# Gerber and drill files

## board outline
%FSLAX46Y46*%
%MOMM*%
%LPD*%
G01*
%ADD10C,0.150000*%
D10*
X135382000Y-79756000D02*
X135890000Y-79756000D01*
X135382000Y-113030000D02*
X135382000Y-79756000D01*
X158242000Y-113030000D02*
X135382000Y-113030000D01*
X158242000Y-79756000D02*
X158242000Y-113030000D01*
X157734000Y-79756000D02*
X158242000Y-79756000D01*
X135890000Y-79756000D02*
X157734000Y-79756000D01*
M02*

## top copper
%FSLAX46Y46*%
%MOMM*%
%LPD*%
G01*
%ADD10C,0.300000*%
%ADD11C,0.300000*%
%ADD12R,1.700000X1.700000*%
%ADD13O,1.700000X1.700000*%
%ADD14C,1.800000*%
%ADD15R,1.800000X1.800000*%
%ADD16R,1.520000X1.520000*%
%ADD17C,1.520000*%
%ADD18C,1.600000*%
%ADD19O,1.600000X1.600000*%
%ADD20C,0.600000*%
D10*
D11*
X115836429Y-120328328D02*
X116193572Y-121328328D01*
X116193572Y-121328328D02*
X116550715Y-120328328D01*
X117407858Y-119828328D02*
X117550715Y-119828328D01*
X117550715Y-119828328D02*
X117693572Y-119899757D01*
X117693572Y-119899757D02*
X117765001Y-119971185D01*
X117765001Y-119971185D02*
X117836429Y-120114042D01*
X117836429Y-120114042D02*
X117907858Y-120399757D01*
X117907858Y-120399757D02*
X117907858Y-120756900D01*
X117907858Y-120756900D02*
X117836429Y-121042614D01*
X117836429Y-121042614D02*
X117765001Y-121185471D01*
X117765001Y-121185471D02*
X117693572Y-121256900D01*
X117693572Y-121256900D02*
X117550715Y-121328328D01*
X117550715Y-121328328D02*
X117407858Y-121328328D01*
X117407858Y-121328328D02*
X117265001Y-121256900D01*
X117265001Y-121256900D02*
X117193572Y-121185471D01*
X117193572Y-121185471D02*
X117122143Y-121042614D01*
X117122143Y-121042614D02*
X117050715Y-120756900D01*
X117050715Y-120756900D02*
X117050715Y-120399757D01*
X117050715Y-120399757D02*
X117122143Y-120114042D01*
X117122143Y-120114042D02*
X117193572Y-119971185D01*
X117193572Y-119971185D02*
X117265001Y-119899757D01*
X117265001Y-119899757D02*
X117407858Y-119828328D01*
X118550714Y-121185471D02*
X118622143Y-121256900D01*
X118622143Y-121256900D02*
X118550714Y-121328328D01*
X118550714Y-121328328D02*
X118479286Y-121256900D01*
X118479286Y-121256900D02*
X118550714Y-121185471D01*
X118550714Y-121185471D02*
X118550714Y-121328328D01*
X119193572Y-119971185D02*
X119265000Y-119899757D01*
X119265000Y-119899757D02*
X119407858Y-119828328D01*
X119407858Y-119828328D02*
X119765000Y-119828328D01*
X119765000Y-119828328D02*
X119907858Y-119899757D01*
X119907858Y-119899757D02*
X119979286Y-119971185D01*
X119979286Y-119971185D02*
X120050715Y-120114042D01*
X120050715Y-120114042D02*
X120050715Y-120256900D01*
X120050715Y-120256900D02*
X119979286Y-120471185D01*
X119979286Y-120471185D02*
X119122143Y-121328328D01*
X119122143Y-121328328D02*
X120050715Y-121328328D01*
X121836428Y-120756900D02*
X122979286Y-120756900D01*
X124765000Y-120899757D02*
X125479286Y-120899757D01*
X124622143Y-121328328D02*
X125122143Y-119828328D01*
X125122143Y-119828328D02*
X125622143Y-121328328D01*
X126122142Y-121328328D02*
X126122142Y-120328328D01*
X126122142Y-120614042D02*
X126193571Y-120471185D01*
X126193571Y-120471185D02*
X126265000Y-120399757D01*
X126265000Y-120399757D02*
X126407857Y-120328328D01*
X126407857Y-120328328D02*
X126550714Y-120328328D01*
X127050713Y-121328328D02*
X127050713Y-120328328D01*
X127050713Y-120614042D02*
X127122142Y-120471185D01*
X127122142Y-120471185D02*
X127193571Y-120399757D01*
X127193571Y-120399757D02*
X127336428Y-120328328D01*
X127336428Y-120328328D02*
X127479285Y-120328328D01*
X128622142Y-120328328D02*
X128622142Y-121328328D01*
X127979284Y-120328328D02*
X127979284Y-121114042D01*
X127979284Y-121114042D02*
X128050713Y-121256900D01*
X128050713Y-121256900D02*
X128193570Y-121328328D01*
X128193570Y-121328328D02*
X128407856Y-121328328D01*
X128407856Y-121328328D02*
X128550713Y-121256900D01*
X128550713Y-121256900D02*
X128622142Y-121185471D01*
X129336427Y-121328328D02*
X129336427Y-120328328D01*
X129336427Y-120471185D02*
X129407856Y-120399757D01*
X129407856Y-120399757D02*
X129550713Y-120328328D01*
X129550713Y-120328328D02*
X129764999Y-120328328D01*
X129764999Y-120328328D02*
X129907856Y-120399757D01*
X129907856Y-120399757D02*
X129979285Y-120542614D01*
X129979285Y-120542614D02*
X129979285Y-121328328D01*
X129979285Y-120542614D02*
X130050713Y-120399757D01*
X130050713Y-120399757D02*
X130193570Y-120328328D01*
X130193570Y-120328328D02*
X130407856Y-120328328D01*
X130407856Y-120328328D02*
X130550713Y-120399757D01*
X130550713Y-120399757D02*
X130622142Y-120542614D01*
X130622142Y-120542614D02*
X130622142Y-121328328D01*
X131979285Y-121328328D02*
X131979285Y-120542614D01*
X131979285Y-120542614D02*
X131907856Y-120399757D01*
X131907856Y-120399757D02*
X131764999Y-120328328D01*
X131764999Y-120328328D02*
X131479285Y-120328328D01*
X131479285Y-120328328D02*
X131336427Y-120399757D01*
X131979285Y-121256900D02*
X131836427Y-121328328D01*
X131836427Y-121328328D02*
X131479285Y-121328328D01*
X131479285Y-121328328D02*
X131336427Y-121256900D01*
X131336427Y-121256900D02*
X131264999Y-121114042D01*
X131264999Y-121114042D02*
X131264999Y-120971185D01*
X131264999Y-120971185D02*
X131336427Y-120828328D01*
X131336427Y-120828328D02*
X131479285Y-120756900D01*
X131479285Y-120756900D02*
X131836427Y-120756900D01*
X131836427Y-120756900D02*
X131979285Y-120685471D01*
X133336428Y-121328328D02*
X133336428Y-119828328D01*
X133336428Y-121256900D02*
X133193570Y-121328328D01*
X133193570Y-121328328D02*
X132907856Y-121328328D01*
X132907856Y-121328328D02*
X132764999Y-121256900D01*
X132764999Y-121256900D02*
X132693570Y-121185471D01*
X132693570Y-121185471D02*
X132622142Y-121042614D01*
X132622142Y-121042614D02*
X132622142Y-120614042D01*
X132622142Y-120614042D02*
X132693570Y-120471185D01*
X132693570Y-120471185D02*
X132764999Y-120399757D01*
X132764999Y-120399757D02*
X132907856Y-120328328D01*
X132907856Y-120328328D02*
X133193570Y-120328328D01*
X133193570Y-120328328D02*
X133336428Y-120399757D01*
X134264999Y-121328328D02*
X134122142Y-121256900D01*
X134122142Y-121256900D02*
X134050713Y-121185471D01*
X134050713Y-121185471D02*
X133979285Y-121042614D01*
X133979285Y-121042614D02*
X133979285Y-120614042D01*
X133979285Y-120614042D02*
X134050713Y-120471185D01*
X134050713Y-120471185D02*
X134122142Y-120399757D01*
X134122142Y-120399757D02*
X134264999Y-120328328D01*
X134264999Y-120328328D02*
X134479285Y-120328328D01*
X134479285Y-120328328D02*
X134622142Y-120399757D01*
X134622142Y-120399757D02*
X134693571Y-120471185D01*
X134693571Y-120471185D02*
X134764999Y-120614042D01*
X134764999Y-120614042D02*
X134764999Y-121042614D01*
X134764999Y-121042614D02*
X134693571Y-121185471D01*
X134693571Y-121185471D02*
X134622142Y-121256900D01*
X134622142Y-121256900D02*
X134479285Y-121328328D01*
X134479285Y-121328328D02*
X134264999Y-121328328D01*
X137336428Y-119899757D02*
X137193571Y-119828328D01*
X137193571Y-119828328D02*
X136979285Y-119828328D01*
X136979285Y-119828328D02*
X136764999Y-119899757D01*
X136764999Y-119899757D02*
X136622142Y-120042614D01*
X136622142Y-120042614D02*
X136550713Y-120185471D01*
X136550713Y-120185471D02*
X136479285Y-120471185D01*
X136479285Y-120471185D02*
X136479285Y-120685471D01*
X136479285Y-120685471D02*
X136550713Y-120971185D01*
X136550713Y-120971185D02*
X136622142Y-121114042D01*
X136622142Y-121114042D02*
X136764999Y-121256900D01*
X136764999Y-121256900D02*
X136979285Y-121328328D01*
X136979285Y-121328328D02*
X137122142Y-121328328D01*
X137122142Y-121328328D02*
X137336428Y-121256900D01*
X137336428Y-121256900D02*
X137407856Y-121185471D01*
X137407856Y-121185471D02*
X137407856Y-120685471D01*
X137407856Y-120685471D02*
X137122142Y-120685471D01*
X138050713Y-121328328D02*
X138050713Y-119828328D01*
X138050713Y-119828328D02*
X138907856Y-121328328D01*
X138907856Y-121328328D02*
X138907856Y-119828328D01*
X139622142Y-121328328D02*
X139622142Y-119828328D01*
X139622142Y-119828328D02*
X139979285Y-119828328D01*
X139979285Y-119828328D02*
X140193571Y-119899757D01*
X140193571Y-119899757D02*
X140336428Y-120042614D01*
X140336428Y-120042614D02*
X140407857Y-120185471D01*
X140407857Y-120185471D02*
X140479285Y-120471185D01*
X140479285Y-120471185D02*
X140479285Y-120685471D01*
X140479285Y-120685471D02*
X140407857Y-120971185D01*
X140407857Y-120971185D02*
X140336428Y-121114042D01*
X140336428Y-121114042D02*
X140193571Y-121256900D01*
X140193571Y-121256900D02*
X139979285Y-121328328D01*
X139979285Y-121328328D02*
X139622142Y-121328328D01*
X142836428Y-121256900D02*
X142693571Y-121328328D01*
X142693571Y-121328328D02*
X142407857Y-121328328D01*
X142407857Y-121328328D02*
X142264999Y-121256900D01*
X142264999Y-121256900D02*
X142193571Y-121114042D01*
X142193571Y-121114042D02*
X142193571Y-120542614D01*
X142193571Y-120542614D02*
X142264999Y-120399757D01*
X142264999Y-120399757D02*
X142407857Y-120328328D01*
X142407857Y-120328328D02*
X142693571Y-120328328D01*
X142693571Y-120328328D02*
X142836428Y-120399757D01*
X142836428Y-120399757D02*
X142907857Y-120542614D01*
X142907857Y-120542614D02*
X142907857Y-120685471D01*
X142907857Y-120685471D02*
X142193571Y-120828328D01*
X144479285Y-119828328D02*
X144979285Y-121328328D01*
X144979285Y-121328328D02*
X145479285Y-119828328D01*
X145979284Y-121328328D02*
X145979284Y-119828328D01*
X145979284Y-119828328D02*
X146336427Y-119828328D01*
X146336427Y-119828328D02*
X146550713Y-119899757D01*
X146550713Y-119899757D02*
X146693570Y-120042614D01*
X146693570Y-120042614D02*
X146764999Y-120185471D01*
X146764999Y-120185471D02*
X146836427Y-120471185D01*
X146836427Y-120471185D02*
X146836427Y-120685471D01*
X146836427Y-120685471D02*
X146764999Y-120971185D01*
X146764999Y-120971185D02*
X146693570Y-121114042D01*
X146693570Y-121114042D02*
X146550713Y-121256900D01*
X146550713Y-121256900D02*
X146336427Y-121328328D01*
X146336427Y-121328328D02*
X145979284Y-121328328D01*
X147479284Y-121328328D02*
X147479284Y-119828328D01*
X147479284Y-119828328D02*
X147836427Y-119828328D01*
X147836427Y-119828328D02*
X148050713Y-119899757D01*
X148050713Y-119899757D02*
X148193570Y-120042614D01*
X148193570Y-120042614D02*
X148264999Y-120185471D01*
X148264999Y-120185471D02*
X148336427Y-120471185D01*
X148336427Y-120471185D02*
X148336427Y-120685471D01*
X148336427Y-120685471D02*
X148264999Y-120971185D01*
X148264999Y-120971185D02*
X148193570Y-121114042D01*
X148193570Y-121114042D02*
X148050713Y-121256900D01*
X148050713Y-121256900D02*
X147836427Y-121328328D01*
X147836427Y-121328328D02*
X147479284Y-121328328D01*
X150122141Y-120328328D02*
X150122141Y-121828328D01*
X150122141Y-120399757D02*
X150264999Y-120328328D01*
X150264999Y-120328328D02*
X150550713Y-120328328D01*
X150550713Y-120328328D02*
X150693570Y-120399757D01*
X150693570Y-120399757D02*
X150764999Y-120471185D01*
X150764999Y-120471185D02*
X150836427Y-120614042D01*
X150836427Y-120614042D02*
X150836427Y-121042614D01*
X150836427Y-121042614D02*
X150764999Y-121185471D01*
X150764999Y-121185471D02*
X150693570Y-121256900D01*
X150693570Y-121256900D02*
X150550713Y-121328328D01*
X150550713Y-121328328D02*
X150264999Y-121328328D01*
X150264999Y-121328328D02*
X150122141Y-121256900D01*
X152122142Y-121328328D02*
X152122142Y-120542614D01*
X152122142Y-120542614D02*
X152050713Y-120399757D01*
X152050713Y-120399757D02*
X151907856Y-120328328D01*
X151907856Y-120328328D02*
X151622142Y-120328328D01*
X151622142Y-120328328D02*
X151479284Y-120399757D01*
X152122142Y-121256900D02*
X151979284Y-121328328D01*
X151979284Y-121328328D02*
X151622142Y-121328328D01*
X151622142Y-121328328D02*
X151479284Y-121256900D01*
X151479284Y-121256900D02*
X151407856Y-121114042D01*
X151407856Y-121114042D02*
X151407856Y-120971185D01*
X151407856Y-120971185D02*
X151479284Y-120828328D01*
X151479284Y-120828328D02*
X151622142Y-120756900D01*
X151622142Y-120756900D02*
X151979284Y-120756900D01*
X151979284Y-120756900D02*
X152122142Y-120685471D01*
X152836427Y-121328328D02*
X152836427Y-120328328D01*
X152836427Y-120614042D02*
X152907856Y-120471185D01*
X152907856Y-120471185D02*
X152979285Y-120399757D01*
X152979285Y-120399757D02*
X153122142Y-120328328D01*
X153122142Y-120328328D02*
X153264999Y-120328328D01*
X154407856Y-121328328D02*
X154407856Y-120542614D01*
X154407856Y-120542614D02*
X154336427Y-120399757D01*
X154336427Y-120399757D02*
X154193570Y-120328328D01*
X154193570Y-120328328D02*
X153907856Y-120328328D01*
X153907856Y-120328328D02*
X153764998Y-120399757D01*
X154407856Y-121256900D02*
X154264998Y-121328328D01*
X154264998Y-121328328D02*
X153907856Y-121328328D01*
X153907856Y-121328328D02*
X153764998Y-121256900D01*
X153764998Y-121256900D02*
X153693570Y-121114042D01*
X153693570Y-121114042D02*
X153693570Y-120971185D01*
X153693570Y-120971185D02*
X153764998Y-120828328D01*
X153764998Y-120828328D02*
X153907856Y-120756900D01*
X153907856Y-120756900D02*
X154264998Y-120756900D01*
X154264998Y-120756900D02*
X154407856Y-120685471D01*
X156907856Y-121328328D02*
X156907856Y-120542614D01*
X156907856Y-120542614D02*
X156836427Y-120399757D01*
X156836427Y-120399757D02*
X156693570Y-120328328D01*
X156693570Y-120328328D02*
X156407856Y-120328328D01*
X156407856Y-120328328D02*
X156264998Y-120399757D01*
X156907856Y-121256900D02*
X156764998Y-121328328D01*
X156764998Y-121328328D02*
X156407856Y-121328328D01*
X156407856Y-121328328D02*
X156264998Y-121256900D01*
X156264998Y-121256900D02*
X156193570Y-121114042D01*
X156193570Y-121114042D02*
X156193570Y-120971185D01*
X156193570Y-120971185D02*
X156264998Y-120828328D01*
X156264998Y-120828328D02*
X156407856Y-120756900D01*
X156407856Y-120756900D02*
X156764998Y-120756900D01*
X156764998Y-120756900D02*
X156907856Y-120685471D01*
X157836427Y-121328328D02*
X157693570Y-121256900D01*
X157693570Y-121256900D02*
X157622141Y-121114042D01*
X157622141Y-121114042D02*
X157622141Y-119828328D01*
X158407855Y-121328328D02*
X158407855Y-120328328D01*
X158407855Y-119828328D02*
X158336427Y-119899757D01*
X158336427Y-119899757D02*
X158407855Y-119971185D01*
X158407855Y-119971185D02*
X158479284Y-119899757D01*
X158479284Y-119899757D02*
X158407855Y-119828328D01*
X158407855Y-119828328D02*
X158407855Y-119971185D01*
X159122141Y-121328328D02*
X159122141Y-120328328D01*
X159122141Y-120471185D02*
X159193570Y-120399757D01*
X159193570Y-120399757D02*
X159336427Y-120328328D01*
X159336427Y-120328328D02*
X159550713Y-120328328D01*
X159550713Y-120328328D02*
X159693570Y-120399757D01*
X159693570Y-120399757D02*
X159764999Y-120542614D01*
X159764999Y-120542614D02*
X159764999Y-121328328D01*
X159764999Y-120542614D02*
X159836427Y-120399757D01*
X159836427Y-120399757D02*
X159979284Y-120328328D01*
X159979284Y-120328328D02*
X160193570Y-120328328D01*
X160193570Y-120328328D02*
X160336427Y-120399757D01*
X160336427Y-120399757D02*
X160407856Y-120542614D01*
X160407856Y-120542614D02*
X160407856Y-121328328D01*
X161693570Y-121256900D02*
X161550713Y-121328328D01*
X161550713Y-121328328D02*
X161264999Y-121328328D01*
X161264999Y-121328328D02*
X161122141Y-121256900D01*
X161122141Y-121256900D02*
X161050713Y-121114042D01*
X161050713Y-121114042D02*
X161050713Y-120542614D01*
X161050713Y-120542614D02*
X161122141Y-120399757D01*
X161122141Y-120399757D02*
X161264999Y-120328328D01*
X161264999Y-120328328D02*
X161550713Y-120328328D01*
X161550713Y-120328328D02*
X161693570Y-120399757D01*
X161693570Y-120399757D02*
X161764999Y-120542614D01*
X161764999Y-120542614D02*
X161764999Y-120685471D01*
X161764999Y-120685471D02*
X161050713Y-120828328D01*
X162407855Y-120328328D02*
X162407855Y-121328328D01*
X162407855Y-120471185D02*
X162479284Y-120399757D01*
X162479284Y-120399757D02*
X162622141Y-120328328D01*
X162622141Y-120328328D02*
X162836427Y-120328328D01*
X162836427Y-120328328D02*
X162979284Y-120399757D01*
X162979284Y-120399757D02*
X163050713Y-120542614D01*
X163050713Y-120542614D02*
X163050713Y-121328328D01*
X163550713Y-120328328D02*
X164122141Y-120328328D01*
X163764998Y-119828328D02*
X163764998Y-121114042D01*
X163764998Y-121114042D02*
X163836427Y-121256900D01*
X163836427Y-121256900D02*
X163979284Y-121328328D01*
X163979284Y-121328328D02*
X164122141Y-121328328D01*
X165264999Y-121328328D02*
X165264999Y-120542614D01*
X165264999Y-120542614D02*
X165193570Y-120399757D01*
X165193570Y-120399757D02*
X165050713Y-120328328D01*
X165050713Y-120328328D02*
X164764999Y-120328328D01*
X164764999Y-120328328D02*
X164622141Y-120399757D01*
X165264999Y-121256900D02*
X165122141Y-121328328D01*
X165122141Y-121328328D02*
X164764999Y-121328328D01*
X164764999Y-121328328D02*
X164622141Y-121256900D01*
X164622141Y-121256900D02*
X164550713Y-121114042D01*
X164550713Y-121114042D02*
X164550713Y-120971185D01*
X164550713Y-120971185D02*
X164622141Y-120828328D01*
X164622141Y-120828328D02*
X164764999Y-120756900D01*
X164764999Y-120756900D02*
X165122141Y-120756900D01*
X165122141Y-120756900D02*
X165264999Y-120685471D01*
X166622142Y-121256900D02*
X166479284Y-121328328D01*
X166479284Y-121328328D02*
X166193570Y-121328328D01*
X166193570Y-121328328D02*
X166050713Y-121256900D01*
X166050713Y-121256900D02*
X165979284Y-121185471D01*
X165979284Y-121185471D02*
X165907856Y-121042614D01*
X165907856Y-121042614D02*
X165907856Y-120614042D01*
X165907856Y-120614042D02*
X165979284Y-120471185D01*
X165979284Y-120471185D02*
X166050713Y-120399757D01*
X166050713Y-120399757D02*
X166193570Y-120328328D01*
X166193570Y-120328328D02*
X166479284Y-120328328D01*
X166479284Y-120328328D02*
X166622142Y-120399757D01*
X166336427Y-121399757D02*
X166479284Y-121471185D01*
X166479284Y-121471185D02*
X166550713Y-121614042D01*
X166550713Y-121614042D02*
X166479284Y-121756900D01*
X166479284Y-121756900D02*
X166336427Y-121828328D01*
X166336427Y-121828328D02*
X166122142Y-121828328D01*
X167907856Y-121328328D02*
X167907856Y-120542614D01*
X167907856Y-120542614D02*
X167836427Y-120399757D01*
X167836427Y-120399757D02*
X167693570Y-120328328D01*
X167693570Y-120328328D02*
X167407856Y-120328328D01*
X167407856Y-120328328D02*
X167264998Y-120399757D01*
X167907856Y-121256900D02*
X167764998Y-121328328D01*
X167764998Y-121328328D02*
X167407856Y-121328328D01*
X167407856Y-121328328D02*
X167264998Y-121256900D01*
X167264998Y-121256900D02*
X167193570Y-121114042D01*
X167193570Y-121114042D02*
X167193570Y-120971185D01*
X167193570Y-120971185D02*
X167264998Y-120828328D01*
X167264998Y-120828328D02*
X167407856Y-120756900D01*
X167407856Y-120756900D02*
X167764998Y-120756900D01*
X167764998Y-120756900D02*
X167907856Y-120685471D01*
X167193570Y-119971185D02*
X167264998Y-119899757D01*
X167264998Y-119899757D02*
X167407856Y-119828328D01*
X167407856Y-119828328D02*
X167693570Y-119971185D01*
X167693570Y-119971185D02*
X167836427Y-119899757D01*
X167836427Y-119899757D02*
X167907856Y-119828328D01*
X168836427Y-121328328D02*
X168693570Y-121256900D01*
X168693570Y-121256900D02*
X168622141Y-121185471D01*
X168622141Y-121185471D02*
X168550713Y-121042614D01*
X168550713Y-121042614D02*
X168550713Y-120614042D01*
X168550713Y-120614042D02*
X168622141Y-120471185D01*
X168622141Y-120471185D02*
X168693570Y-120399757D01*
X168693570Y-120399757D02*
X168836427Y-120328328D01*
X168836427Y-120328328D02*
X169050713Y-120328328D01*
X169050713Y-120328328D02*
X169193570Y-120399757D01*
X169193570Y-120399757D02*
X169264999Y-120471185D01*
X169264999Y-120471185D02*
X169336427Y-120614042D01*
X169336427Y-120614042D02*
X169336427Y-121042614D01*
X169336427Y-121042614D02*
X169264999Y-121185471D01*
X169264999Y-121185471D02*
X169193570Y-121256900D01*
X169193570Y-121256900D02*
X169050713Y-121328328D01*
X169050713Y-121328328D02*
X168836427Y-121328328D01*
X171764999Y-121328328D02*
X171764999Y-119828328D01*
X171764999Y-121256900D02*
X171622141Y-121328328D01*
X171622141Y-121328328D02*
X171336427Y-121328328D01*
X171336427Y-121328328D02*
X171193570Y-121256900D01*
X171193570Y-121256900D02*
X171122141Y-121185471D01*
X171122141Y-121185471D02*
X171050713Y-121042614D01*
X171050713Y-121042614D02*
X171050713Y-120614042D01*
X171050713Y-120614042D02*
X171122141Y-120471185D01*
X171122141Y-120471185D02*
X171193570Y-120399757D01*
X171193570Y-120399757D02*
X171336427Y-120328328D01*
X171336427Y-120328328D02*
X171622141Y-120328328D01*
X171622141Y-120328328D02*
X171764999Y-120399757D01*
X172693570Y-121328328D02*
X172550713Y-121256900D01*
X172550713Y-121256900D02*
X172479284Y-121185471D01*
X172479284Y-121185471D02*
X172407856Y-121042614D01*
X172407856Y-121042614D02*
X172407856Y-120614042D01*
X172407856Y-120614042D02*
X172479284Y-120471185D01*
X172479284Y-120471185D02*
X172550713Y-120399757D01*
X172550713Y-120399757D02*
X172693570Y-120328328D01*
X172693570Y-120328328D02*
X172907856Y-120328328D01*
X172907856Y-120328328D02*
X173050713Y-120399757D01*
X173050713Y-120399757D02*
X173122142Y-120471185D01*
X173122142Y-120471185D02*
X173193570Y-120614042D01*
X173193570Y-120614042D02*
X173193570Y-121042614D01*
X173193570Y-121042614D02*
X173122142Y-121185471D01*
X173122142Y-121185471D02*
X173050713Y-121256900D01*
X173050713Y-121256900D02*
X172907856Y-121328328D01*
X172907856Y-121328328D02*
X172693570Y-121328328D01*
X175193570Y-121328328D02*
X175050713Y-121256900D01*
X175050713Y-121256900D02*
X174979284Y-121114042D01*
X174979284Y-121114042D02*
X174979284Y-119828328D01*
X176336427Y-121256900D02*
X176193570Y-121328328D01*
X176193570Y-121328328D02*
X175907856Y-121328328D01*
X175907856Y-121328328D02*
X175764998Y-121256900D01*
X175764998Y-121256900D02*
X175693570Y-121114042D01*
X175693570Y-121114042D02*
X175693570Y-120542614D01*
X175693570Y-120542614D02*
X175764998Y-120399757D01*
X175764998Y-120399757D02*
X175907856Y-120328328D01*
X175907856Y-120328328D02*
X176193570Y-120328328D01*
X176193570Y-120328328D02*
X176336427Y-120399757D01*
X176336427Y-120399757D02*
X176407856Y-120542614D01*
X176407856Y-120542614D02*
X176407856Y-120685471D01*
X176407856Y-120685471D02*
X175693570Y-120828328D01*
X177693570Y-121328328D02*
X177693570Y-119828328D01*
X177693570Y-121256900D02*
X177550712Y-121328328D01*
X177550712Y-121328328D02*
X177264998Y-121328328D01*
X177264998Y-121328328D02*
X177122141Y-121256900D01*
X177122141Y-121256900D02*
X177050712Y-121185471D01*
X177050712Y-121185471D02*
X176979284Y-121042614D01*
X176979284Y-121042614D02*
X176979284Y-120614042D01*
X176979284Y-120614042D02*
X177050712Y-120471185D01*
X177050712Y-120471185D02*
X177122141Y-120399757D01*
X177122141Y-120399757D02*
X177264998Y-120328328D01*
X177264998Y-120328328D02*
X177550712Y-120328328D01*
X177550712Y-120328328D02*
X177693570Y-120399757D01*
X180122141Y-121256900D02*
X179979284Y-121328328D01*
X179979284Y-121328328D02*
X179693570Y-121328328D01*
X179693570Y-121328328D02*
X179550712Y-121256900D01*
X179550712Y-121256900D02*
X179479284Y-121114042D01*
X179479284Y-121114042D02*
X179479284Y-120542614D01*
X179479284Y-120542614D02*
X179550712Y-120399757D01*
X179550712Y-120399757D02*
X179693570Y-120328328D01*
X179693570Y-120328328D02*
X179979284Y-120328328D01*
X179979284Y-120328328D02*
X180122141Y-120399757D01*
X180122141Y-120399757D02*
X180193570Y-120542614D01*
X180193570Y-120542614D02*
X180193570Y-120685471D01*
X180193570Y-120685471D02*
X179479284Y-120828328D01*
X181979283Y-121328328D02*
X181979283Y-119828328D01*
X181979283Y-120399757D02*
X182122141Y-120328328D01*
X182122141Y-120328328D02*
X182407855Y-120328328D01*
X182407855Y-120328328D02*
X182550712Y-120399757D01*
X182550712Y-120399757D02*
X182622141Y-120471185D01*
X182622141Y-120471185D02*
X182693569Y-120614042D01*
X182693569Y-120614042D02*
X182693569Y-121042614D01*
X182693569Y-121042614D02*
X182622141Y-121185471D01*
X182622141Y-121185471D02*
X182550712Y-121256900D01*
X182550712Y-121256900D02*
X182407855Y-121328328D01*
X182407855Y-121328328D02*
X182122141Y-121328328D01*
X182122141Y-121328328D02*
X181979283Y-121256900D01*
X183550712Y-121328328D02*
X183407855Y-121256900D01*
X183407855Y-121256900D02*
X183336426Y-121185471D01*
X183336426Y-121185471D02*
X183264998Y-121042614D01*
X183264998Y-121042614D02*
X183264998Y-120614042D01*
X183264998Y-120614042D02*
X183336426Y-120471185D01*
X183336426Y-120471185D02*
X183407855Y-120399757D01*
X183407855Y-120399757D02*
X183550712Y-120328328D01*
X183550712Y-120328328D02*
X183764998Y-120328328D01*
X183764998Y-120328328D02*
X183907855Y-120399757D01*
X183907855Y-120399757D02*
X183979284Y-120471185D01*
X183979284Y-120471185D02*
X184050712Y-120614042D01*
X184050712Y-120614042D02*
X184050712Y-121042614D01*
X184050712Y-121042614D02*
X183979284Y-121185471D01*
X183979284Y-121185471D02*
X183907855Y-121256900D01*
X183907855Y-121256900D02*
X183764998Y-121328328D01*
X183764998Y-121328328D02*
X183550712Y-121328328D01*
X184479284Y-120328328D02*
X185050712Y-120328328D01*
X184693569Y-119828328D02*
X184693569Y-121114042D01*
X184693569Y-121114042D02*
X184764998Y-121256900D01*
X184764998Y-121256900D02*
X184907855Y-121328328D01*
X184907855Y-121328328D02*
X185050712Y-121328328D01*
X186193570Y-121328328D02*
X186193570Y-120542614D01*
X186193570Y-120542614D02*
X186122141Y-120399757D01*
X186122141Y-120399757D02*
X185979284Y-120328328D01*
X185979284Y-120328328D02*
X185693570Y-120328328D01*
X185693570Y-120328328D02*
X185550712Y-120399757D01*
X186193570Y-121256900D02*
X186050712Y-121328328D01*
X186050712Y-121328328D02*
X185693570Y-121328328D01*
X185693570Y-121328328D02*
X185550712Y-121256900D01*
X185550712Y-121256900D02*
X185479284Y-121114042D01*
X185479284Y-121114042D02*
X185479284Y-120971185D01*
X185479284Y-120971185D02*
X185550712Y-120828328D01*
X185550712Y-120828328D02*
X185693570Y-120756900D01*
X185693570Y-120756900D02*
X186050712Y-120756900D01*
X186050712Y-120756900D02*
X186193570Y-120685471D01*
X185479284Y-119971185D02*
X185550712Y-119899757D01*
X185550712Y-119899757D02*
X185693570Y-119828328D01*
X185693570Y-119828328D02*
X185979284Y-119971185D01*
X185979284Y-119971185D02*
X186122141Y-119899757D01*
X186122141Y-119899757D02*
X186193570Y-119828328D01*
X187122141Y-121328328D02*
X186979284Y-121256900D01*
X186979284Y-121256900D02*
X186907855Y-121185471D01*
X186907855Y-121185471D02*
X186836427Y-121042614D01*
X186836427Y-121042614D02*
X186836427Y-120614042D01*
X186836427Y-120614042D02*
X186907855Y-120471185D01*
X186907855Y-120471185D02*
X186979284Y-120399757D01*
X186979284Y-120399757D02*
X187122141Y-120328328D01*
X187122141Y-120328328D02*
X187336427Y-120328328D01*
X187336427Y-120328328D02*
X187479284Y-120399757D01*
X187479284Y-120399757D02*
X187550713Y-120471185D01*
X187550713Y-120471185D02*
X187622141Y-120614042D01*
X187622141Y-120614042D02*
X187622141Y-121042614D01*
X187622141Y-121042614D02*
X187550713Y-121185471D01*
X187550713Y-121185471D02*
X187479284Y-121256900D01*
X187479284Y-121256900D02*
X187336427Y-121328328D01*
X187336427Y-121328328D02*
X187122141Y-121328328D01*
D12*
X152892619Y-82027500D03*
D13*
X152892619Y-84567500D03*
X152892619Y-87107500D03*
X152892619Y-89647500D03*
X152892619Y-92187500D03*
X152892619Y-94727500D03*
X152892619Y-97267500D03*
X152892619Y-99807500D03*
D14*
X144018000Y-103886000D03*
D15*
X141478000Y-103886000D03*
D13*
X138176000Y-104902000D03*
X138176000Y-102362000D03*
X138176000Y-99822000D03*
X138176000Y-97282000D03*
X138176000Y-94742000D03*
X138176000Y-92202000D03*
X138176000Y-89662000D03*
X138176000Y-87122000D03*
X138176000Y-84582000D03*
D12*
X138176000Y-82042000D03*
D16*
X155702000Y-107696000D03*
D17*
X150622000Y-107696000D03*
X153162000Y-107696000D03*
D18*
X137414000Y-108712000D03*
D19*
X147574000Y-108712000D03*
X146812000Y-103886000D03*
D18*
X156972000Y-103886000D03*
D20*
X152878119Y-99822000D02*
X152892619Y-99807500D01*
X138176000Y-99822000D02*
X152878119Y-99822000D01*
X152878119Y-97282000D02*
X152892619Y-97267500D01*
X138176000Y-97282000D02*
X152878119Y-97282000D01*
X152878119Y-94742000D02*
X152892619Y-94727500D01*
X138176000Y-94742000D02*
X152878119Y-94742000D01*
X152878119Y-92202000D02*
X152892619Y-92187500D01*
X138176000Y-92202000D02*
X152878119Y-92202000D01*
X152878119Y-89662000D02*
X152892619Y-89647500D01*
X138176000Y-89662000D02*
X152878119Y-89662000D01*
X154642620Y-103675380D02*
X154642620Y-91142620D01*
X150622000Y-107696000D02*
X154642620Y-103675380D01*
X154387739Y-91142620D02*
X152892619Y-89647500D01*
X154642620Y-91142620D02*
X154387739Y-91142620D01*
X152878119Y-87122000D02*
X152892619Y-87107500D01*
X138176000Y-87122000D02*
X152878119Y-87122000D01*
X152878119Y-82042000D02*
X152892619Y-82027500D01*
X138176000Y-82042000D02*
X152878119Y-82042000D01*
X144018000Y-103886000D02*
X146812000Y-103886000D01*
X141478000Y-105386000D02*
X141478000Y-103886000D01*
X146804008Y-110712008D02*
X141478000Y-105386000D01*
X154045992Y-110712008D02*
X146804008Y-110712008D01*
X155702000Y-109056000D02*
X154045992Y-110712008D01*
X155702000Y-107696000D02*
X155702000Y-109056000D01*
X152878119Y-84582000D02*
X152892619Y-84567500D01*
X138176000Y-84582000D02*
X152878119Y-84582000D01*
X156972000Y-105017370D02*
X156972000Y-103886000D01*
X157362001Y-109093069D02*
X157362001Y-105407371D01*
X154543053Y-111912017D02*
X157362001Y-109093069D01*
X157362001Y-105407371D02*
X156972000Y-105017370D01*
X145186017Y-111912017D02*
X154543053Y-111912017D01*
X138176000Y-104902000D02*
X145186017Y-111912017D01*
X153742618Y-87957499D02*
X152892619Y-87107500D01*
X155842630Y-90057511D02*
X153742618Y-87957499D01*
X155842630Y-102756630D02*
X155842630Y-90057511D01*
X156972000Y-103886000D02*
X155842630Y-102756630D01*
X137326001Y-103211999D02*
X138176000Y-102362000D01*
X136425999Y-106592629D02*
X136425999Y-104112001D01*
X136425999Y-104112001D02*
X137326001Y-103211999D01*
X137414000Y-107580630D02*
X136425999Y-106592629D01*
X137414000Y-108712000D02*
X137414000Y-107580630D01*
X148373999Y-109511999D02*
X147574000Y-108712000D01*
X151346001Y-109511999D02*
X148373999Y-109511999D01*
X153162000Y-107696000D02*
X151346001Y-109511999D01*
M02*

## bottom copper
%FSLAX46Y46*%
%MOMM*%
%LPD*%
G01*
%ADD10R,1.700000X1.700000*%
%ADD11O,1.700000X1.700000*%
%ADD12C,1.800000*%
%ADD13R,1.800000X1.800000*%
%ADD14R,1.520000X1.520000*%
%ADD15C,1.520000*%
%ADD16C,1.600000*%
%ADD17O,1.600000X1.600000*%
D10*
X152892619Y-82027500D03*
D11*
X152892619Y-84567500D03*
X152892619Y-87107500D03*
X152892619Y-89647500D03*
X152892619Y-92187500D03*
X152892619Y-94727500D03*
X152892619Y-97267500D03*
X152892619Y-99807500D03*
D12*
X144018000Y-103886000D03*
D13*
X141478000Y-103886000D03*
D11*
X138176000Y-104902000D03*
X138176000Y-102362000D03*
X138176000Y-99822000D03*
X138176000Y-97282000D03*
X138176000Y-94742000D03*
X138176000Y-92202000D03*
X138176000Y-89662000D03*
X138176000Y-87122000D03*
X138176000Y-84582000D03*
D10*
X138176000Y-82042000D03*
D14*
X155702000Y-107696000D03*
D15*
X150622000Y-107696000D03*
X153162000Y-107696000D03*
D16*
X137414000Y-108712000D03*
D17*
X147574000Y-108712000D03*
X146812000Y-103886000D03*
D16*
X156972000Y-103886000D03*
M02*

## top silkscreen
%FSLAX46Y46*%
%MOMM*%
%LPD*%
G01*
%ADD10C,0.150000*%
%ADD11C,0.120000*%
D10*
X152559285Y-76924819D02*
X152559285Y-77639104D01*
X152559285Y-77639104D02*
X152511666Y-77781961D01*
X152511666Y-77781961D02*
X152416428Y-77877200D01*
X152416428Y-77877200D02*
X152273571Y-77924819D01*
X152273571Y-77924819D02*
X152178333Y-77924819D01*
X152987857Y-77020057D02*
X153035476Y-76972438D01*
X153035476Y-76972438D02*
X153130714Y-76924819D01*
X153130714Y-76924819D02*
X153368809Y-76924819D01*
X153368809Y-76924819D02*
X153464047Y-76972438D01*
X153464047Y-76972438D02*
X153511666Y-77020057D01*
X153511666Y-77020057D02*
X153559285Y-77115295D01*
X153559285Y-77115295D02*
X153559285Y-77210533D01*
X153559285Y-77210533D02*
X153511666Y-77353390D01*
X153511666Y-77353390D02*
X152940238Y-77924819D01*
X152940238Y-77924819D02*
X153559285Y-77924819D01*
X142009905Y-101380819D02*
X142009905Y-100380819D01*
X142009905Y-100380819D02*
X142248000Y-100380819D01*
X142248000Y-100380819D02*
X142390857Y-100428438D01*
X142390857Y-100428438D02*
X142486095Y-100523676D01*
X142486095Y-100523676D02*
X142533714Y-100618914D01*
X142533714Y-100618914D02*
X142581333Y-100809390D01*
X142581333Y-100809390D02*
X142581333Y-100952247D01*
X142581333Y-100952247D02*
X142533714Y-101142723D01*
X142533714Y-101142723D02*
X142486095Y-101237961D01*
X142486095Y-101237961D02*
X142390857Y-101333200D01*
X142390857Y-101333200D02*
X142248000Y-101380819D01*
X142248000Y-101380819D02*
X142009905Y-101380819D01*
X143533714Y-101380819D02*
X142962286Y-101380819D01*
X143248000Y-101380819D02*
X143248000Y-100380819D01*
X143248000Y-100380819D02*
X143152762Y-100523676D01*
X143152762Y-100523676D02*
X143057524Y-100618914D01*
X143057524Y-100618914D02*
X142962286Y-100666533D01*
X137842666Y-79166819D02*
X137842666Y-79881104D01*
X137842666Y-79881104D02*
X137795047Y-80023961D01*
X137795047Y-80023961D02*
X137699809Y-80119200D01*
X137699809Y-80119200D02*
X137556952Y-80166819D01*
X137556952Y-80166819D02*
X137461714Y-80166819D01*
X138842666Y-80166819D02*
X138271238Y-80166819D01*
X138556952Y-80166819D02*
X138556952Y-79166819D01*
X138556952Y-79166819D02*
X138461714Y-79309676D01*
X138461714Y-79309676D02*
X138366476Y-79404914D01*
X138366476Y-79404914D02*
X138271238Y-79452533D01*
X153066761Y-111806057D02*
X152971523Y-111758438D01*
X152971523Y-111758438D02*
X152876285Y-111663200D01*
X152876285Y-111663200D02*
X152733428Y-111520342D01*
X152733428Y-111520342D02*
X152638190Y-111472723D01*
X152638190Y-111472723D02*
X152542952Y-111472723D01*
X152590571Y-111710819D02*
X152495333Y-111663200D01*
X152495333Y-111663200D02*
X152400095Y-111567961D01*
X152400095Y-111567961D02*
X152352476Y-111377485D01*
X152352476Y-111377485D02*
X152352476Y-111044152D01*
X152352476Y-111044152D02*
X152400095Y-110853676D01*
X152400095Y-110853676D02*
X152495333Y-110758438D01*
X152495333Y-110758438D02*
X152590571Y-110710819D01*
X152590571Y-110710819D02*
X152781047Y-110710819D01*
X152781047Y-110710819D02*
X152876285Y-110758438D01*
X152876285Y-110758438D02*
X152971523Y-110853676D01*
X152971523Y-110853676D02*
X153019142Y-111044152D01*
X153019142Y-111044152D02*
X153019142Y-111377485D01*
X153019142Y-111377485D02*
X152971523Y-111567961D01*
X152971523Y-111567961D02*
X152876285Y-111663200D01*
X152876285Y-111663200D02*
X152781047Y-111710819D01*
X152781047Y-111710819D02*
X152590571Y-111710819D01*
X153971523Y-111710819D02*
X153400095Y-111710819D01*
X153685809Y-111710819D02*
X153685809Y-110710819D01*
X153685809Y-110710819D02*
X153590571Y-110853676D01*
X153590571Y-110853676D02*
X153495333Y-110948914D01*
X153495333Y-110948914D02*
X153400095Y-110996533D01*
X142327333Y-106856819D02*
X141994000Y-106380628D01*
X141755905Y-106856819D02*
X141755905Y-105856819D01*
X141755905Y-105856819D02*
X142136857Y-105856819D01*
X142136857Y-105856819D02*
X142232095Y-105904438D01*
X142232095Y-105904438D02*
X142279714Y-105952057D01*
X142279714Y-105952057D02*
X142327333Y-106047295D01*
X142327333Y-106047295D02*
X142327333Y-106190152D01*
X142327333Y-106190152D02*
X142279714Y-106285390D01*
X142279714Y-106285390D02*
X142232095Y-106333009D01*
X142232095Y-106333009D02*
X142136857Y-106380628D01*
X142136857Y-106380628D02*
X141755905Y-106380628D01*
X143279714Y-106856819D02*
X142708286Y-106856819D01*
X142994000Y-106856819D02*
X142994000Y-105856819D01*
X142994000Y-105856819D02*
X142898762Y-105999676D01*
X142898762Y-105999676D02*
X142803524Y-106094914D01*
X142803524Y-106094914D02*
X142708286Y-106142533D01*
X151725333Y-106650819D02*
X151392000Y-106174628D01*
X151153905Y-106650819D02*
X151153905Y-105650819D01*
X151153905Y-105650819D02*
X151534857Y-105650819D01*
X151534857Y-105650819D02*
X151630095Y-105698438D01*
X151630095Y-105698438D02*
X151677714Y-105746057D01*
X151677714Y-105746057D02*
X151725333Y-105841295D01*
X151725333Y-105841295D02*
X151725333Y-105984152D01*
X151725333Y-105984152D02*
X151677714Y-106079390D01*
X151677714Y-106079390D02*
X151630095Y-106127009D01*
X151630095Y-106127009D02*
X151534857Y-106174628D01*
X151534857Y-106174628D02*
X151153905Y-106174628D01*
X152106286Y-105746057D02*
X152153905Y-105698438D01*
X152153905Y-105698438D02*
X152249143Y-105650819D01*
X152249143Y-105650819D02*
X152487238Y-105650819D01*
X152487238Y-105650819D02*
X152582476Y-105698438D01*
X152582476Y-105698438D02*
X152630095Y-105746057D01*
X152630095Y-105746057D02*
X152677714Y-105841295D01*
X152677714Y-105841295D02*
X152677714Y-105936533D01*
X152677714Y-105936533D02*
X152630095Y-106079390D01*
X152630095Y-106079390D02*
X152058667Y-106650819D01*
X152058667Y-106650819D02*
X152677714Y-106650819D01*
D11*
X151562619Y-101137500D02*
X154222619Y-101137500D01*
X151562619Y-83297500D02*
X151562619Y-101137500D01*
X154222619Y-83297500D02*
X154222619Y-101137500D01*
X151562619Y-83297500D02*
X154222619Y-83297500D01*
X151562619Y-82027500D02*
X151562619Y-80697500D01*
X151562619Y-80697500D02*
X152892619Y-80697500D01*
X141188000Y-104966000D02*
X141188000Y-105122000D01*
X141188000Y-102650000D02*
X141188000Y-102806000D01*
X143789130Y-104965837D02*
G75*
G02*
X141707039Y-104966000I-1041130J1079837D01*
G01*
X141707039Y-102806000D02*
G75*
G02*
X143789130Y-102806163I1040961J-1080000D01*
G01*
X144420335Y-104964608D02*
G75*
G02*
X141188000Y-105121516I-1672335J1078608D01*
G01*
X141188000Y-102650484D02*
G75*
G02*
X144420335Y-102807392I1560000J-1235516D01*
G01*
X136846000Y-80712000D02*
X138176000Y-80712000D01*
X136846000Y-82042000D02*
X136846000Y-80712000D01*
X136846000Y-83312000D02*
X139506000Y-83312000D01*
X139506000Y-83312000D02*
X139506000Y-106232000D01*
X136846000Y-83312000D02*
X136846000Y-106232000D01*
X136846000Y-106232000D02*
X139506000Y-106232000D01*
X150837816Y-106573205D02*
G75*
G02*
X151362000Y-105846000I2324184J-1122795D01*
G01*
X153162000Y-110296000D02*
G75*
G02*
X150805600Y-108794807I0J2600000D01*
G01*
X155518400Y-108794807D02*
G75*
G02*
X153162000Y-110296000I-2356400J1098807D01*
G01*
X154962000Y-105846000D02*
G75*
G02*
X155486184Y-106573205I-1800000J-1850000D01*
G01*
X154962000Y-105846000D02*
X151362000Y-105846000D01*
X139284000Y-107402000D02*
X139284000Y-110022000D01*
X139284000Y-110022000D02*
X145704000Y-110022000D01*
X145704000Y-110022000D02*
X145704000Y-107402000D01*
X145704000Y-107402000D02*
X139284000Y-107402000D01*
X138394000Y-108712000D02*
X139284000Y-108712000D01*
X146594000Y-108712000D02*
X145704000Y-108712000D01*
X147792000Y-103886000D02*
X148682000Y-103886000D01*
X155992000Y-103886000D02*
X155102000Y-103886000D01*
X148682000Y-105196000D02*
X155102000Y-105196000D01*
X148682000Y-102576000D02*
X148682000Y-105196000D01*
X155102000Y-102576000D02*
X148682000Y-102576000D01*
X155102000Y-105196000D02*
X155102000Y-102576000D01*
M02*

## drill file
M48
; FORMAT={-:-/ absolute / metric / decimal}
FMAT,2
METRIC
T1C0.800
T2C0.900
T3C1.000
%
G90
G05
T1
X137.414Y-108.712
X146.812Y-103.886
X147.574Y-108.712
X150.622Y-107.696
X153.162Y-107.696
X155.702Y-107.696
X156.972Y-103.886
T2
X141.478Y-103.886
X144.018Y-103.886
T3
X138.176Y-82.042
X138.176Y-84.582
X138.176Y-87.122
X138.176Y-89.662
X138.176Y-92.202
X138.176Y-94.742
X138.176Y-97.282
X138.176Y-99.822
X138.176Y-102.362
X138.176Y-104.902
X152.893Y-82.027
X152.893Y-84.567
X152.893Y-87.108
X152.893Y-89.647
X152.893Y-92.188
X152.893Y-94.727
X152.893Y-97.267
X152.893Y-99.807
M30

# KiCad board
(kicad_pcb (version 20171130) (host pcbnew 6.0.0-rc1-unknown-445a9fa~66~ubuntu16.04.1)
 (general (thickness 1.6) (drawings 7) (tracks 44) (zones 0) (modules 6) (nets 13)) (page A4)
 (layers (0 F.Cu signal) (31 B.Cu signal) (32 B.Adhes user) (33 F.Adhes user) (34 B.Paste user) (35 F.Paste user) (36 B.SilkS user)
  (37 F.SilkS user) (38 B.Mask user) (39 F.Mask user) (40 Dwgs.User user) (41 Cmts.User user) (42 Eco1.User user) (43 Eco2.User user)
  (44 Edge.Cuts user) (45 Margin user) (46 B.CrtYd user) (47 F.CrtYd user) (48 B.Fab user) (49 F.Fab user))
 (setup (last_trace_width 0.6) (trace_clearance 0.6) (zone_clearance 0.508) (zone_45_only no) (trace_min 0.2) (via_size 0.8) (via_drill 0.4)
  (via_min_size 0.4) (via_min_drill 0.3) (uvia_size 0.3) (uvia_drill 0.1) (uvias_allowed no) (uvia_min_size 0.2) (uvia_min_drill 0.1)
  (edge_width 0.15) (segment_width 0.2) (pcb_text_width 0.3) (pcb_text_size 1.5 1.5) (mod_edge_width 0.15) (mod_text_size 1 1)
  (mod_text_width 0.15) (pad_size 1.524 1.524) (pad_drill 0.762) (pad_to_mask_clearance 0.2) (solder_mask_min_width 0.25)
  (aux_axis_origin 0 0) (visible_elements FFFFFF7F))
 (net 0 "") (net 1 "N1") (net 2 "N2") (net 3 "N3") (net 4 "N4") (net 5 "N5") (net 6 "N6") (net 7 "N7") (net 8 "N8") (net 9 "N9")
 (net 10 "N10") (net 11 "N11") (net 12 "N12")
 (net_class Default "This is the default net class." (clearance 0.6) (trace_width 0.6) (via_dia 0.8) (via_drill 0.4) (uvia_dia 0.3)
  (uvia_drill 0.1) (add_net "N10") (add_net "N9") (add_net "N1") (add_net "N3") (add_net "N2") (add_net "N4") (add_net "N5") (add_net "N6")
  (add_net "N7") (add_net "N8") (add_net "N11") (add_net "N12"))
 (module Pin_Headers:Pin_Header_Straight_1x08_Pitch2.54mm (layer F.Cu) (at 152.892619 82.0275)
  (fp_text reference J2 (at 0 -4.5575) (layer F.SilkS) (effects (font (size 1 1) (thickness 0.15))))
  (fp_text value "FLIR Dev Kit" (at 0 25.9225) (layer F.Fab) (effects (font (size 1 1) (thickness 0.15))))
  (fp_line (start -1.33 19.11) (end 1.33 19.11) (layer F.SilkS) (width 0.12))
  (fp_line (start -1.33 1.27) (end -1.33 19.11) (layer F.SilkS) (width 0.12))
  (fp_line (start 1.33 1.27) (end 1.33 19.11) (layer F.SilkS) (width 0.12))
  (fp_line (start -1.33 1.27) (end 1.33 1.27) (layer F.SilkS) (width 0.12))
  (fp_line (start -1.33 0) (end -1.33 -1.33) (layer F.SilkS) (width 0.12))
  (fp_line (start -1.33 -1.33) (end 0 -1.33) (layer F.SilkS) (width 0.12))
  (pad 1 thru_hole rect (at 0 0) (size 1.7 1.7) (drill 1) (layers *.Cu *.Mask) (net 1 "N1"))
  (pad 2 thru_hole oval (at 0 2.54) (size 1.7 1.7) (drill 1) (layers *.Cu *.Mask) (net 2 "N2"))
  (pad 3 thru_hole oval (at 0 5.08) (size 1.7 1.7) (drill 1) (layers *.Cu *.Mask) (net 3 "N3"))
  (pad 4 thru_hole oval (at 0 7.62) (size 1.7 1.7) (drill 1) (layers *.Cu *.Mask) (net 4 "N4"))
  (pad 5 thru_hole oval (at 0 10.16) (size 1.7 1.7) (drill 1) (layers *.Cu *.Mask) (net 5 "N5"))
  (pad 6 thru_hole oval (at 0 12.7) (size 1.7 1.7) (drill 1) (layers *.Cu *.Mask) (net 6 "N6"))
  (pad 7 thru_hole oval (at 0 15.24) (size 1.7 1.7) (drill 1) (layers *.Cu *.Mask) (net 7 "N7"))
  (pad 8 thru_hole oval (at 0 17.78) (size 1.7 1.7) (drill 1) (layers *.Cu *.Mask) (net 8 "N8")))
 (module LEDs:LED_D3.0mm (layer F.Cu) (at 141.478 103.886)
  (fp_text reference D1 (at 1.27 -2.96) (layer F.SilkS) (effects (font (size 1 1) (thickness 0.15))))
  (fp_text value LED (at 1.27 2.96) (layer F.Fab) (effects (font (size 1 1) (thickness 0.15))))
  (fp_line (start -0.29 1.08) (end -0.29 1.236) (layer F.SilkS) (width 0.12))
  (fp_line (start -0.29 -1.236) (end -0.29 -1.08) (layer F.SilkS) (width 0.12))
  (fp_arc (start 1.27 0) (end 0.229039 1.08) (angle -87.9) (layer F.SilkS) (width 0.12))
  (fp_arc (start 1.27 0) (end 0.229039 -1.08) (angle 87.9) (layer F.SilkS) (width 0.12))
  (fp_arc (start 1.27 0) (end -0.29 1.235516) (angle -108.8) (layer F.SilkS) (width 0.12))
  (fp_arc (start 1.27 0) (end -0.29 -1.235516) (angle 108.8) (layer F.SilkS) (width 0.12))
  (pad 2 thru_hole circle (at 2.54 0) (size 1.8 1.8) (drill 0.9) (layers *.Cu *.Mask) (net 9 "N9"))
  (pad 1 thru_hole rect (at 0 0) (size 1.8 1.8) (drill 0.9) (layers *.Cu *.Mask) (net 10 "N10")))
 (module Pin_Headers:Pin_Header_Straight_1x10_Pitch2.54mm (layer F.Cu) (at 138.176 82.042)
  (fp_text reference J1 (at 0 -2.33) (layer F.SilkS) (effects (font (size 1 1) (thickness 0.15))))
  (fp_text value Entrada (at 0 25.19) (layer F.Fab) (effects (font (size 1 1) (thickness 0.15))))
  (fp_line (start -1.33 -1.33) (end 0 -1.33) (layer F.SilkS) (width 0.12))
  (fp_line (start -1.33 0) (end -1.33 -1.33) (layer F.SilkS) (width 0.12))
  (fp_line (start -1.33 1.27) (end 1.33 1.27) (layer F.SilkS) (width 0.12))
  (fp_line (start 1.33 1.27) (end 1.33 24.19) (layer F.SilkS) (width 0.12))
  (fp_line (start -1.33 1.27) (end -1.33 24.19) (layer F.SilkS) (width 0.12))
  (fp_line (start -1.33 24.19) (end 1.33 24.19) (layer F.SilkS) (width 0.12))
  (pad 10 thru_hole oval (at 0 22.86) (size 1.7 1.7) (drill 1) (layers *.Cu *.Mask) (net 3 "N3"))
  (pad 9 thru_hole oval (at 0 20.32) (size 1.7 1.7) (drill 1) (layers *.Cu *.Mask) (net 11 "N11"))
  (pad 8 thru_hole oval (at 0 17.78) (size 1.7 1.7) (drill 1) (layers *.Cu *.Mask) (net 8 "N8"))
  (pad 7 thru_hole oval (at 0 15.24) (size 1.7 1.7) (drill 1) (layers *.Cu *.Mask) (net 7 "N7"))
  (pad 6 thru_hole oval (at 0 12.7) (size 1.7 1.7) (drill 1) (layers *.Cu *.Mask) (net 6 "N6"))
  (pad 5 thru_hole oval (at 0 10.16) (size 1.7 1.7) (drill 1) (layers *.Cu *.Mask) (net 5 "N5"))
  (pad 4 thru_hole oval (at 0 7.62) (size 1.7 1.7) (drill 1) (layers *.Cu *.Mask) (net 4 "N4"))
  (pad 3 thru_hole oval (at 0 5.08) (size 1.7 1.7) (drill 1) (layers *.Cu *.Mask) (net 3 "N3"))
  (pad 2 thru_hole oval (at 0 2.54) (size 1.7 1.7) (drill 1) (layers *.Cu *.Mask) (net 2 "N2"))
  (pad 1 thru_hole rect (at 0 0) (size 1.7 1.7) (drill 1) (layers *.Cu *.Mask) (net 1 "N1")))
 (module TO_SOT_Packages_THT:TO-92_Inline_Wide (layer F.Cu) (at 155.702 107.696 180)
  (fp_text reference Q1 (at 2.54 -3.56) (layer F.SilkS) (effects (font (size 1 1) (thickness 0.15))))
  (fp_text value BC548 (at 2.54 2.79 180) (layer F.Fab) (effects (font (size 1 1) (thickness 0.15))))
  (fp_arc (start 2.54 0) (end 4.34 1.85) (angle -20) (layer F.SilkS) (width 0.12))
  (fp_arc (start 2.54 0) (end 2.54 -2.6) (angle 65) (layer F.SilkS) (width 0.12))
  (fp_arc (start 2.54 0) (end 2.54 -2.6) (angle -65) (layer F.SilkS) (width 0.12))
  (fp_arc (start 2.54 0) (end 0.74 1.85) (angle 20) (layer F.SilkS) (width 0.12))
  (fp_line (start 0.74 1.85) (end 4.34 1.85) (layer F.SilkS) (width 0.12))
  (pad 1 thru_hole rect (at 0 0 270) (size 1.52 1.52) (drill 0.8) (layers *.Cu *.Mask) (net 10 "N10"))
  (pad 3 thru_hole circle (at 5.08 0 270) (size 1.52 1.52) (drill 0.8) (layers *.Cu *.Mask) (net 4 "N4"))
  (pad 2 thru_hole circle (at 2.54 0 270) (size 1.52 1.52) (drill 0.8) (layers *.Cu *.Mask) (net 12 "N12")))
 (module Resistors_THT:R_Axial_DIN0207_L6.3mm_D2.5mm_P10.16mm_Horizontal (layer F.Cu) (at 137.414 108.712)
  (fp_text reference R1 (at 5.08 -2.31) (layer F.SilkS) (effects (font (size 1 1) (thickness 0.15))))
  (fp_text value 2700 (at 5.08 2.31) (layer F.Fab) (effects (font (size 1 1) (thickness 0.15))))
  (fp_line (start 1.87 -1.31) (end 1.87 1.31) (layer F.SilkS) (width 0.12))
  (fp_line (start 1.87 1.31) (end 8.29 1.31) (layer F.SilkS) (width 0.12))
  (fp_line (start 8.29 1.31) (end 8.29 -1.31) (layer F.SilkS) (width 0.12))
  (fp_line (start 8.29 -1.31) (end 1.87 -1.31) (layer F.SilkS) (width 0.12))
  (fp_line (start 0.98 0) (end 1.87 0) (layer F.SilkS) (width 0.12))
  (fp_line (start 9.18 0) (end 8.29 0) (layer F.SilkS) (width 0.12))
  (pad 1 thru_hole circle (at 0 0) (size 1.6 1.6) (drill 0.8) (layers *.Cu *.Mask) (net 11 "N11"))
  (pad 2 thru_hole oval (at 10.16 0) (size 1.6 1.6) (drill 0.8) (layers *.Cu *.Mask) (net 12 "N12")))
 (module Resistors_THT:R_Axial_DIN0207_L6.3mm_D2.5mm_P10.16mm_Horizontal (layer F.Cu) (at 156.972 103.886 180)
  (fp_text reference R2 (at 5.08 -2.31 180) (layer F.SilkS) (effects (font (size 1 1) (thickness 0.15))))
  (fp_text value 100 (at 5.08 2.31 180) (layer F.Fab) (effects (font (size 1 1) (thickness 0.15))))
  (fp_line (start 9.18 0) (end 8.29 0) (layer F.SilkS) (width 0.12))
  (fp_line (start 0.98 0) (end 1.87 0) (layer F.SilkS) (width 0.12))
  (fp_line (start 8.29 -1.31) (end 1.87 -1.31) (layer F.SilkS) (width 0.12))
  (fp_line (start 8.29 1.31) (end 8.29 -1.31) (layer F.SilkS) (width 0.12))
  (fp_line (start 1.87 1.31) (end 8.29 1.31) (layer F.SilkS) (width 0.12))
  (fp_line (start 1.87 -1.31) (end 1.87 1.31) (layer F.SilkS) (width 0.12))
  (pad 2 thru_hole oval (at 10.16 0 180) (size 1.6 1.6) (drill 0.8) (layers *.Cu *.Mask) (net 9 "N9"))
  (pad 1 thru_hole circle (at 0 0 180) (size 1.6 1.6) (drill 0.8) (layers *.Cu *.Mask) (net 3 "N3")))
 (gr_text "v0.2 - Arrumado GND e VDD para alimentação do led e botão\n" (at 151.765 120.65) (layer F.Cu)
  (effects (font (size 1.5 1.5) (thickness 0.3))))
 (gr_line (start 135.382 79.756) (end 135.89 79.756) (layer Edge.Cuts) (width 0.15))
 (gr_line (start 135.382 113.03) (end 135.382 79.756) (layer Edge.Cuts) (width 0.15))
 (gr_line (start 158.242 113.03) (end 135.382 113.03) (layer Edge.Cuts) (width 0.15))
 (gr_line (start 158.242 79.756) (end 158.242 113.03) (layer Edge.Cuts) (width 0.15))
 (gr_line (start 157.734 79.756) (end 158.242 79.756) (layer Edge.Cuts) (width 0.15))
 (gr_line (start 135.89 79.756) (end 157.734 79.756) (layer Edge.Cuts) (width 0.15))
 (segment (start 152.878119 99.822) (end 152.892619 99.8075) (width 0.6) (layer F.Cu) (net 8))
 (segment (start 138.176 99.822) (end 152.878119 99.822) (width 0.6) (layer F.Cu) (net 8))
 (segment (start 152.878119 97.282) (end 152.892619 97.2675) (width 0.6) (layer F.Cu) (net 7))
 (segment (start 138.176 97.282) (end 152.878119 97.282) (width 0.6) (layer F.Cu) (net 7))
 (segment (start 152.878119 94.742) (end 152.892619 94.7275) (width 0.6) (layer F.Cu) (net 6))
 (segment (start 138.176 94.742) (end 152.878119 94.742) (width 0.6) (layer F.Cu) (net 6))
 (segment (start 152.878119 92.202) (end 152.892619 92.1875) (width 0.6) (layer F.Cu) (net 5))
 (segment (start 138.176 92.202) (end 152.878119 92.202) (width 0.6) (layer F.Cu) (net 5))
 (segment (start 152.878119 89.662) (end 152.892619 89.6475) (width 0.6) (layer F.Cu) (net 4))
 (segment (start 138.176 89.662) (end 152.878119 89.662) (width 0.6) (layer F.Cu) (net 4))
 (segment (start 154.64262 103.67538) (end 154.64262 91.14262) (width 0.6) (layer F.Cu) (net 4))
 (segment (start 150.622 107.696) (end 154.64262 103.67538) (width 0.6) (layer F.Cu) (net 4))
 (segment (start 154.387739 91.14262) (end 152.892619 89.6475) (width 0.6) (layer F.Cu) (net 4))
 (segment (start 154.64262 91.14262) (end 154.387739 91.14262) (width 0.6) (layer F.Cu) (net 4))
 (segment (start 152.878119 87.122) (end 152.892619 87.1075) (width 0.6) (layer F.Cu) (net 3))
 (segment (start 138.176 87.122) (end 152.878119 87.122) (width 0.6) (layer F.Cu) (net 3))
 (segment (start 152.878119 82.042) (end 152.892619 82.0275) (width 0.6) (layer F.Cu) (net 1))
 (segment (start 138.176 82.042) (end 152.878119 82.042) (width 0.6) (layer F.Cu) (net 1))
 (segment (start 144.018 103.886) (end 146.812 103.886) (width 0.6) (layer F.Cu) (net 9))
 (segment (start 141.478 105.386) (end 141.478 103.886) (width 0.6) (layer F.Cu) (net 10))
 (segment (start 146.804008 110.712008) (end 141.478 105.386) (width 0.6) (layer F.Cu) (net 10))
 (segment (start 154.045992 110.712008) (end 146.804008 110.712008) (width 0.6) (layer F.Cu) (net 10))
 (segment (start 155.702 109.056) (end 154.045992 110.712008) (width 0.6) (layer F.Cu) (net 10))
 (segment (start 155.702 107.696) (end 155.702 109.056) (width 0.6) (layer F.Cu) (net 10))
 (segment (start 152.878119 84.582) (end 152.892619 84.5675) (width 0.6) (layer F.Cu) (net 2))
 (segment (start 138.176 84.582) (end 152.878119 84.582) (width 0.6) (layer F.Cu) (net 2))
 (segment (start 156.972 105.01737) (end 156.972 103.886) (width 0.6) (layer F.Cu) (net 3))
 (segment (start 157.362001 109.093069) (end 157.362001 105.407371) (width 0.6) (layer F.Cu) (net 3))
 (segment (start 154.543053 111.912017) (end 157.362001 109.093069) (width 0.6) (layer F.Cu) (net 3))
 (segment (start 157.362001 105.407371) (end 156.972 105.01737) (width 0.6) (layer F.Cu) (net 3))
 (segment (start 145.186017 111.912017) (end 154.543053 111.912017) (width 0.6) (layer F.Cu) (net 3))
 (segment (start 138.176 104.902) (end 145.186017 111.912017) (width 0.6) (layer F.Cu) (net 3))
 (segment (start 153.742618 87.957499) (end 152.892619 87.1075) (width 0.6) (layer F.Cu) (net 3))
 (segment (start 155.84263 90.057511) (end 153.742618 87.957499) (width 0.6) (layer F.Cu) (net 3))
 (segment (start 155.84263 102.75663) (end 155.84263 90.057511) (width 0.6) (layer F.Cu) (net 3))
 (segment (start 156.972 103.886) (end 155.84263 102.75663) (width 0.6) (layer F.Cu) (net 3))
 (segment (start 137.326001 103.211999) (end 138.176 102.362) (width 0.6) (layer F.Cu) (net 11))
 (segment (start 136.425999 106.592629) (end 136.425999 104.112001) (width 0.6) (layer F.Cu) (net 11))
 (segment (start 136.425999 104.112001) (end 137.326001 103.211999) (width 0.6) (layer F.Cu) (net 11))
 (segment (start 137.414 107.58063) (end 136.425999 106.592629) (width 0.6) (layer F.Cu) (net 11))
 (segment (start 137.414 108.712) (end 137.414 107.58063) (width 0.6) (layer F.Cu) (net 11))
 (segment (start 148.373999 109.511999) (end 147.574 108.712) (width 0.6) (layer F.Cu) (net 12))
 (segment (start 151.346001 109.511999) (end 148.373999 109.511999) (width 0.6) (layer F.Cu) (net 12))
 (segment (start 153.162 107.696) (end 151.346001 109.511999) (width 0.6) (layer F.Cu) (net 12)))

